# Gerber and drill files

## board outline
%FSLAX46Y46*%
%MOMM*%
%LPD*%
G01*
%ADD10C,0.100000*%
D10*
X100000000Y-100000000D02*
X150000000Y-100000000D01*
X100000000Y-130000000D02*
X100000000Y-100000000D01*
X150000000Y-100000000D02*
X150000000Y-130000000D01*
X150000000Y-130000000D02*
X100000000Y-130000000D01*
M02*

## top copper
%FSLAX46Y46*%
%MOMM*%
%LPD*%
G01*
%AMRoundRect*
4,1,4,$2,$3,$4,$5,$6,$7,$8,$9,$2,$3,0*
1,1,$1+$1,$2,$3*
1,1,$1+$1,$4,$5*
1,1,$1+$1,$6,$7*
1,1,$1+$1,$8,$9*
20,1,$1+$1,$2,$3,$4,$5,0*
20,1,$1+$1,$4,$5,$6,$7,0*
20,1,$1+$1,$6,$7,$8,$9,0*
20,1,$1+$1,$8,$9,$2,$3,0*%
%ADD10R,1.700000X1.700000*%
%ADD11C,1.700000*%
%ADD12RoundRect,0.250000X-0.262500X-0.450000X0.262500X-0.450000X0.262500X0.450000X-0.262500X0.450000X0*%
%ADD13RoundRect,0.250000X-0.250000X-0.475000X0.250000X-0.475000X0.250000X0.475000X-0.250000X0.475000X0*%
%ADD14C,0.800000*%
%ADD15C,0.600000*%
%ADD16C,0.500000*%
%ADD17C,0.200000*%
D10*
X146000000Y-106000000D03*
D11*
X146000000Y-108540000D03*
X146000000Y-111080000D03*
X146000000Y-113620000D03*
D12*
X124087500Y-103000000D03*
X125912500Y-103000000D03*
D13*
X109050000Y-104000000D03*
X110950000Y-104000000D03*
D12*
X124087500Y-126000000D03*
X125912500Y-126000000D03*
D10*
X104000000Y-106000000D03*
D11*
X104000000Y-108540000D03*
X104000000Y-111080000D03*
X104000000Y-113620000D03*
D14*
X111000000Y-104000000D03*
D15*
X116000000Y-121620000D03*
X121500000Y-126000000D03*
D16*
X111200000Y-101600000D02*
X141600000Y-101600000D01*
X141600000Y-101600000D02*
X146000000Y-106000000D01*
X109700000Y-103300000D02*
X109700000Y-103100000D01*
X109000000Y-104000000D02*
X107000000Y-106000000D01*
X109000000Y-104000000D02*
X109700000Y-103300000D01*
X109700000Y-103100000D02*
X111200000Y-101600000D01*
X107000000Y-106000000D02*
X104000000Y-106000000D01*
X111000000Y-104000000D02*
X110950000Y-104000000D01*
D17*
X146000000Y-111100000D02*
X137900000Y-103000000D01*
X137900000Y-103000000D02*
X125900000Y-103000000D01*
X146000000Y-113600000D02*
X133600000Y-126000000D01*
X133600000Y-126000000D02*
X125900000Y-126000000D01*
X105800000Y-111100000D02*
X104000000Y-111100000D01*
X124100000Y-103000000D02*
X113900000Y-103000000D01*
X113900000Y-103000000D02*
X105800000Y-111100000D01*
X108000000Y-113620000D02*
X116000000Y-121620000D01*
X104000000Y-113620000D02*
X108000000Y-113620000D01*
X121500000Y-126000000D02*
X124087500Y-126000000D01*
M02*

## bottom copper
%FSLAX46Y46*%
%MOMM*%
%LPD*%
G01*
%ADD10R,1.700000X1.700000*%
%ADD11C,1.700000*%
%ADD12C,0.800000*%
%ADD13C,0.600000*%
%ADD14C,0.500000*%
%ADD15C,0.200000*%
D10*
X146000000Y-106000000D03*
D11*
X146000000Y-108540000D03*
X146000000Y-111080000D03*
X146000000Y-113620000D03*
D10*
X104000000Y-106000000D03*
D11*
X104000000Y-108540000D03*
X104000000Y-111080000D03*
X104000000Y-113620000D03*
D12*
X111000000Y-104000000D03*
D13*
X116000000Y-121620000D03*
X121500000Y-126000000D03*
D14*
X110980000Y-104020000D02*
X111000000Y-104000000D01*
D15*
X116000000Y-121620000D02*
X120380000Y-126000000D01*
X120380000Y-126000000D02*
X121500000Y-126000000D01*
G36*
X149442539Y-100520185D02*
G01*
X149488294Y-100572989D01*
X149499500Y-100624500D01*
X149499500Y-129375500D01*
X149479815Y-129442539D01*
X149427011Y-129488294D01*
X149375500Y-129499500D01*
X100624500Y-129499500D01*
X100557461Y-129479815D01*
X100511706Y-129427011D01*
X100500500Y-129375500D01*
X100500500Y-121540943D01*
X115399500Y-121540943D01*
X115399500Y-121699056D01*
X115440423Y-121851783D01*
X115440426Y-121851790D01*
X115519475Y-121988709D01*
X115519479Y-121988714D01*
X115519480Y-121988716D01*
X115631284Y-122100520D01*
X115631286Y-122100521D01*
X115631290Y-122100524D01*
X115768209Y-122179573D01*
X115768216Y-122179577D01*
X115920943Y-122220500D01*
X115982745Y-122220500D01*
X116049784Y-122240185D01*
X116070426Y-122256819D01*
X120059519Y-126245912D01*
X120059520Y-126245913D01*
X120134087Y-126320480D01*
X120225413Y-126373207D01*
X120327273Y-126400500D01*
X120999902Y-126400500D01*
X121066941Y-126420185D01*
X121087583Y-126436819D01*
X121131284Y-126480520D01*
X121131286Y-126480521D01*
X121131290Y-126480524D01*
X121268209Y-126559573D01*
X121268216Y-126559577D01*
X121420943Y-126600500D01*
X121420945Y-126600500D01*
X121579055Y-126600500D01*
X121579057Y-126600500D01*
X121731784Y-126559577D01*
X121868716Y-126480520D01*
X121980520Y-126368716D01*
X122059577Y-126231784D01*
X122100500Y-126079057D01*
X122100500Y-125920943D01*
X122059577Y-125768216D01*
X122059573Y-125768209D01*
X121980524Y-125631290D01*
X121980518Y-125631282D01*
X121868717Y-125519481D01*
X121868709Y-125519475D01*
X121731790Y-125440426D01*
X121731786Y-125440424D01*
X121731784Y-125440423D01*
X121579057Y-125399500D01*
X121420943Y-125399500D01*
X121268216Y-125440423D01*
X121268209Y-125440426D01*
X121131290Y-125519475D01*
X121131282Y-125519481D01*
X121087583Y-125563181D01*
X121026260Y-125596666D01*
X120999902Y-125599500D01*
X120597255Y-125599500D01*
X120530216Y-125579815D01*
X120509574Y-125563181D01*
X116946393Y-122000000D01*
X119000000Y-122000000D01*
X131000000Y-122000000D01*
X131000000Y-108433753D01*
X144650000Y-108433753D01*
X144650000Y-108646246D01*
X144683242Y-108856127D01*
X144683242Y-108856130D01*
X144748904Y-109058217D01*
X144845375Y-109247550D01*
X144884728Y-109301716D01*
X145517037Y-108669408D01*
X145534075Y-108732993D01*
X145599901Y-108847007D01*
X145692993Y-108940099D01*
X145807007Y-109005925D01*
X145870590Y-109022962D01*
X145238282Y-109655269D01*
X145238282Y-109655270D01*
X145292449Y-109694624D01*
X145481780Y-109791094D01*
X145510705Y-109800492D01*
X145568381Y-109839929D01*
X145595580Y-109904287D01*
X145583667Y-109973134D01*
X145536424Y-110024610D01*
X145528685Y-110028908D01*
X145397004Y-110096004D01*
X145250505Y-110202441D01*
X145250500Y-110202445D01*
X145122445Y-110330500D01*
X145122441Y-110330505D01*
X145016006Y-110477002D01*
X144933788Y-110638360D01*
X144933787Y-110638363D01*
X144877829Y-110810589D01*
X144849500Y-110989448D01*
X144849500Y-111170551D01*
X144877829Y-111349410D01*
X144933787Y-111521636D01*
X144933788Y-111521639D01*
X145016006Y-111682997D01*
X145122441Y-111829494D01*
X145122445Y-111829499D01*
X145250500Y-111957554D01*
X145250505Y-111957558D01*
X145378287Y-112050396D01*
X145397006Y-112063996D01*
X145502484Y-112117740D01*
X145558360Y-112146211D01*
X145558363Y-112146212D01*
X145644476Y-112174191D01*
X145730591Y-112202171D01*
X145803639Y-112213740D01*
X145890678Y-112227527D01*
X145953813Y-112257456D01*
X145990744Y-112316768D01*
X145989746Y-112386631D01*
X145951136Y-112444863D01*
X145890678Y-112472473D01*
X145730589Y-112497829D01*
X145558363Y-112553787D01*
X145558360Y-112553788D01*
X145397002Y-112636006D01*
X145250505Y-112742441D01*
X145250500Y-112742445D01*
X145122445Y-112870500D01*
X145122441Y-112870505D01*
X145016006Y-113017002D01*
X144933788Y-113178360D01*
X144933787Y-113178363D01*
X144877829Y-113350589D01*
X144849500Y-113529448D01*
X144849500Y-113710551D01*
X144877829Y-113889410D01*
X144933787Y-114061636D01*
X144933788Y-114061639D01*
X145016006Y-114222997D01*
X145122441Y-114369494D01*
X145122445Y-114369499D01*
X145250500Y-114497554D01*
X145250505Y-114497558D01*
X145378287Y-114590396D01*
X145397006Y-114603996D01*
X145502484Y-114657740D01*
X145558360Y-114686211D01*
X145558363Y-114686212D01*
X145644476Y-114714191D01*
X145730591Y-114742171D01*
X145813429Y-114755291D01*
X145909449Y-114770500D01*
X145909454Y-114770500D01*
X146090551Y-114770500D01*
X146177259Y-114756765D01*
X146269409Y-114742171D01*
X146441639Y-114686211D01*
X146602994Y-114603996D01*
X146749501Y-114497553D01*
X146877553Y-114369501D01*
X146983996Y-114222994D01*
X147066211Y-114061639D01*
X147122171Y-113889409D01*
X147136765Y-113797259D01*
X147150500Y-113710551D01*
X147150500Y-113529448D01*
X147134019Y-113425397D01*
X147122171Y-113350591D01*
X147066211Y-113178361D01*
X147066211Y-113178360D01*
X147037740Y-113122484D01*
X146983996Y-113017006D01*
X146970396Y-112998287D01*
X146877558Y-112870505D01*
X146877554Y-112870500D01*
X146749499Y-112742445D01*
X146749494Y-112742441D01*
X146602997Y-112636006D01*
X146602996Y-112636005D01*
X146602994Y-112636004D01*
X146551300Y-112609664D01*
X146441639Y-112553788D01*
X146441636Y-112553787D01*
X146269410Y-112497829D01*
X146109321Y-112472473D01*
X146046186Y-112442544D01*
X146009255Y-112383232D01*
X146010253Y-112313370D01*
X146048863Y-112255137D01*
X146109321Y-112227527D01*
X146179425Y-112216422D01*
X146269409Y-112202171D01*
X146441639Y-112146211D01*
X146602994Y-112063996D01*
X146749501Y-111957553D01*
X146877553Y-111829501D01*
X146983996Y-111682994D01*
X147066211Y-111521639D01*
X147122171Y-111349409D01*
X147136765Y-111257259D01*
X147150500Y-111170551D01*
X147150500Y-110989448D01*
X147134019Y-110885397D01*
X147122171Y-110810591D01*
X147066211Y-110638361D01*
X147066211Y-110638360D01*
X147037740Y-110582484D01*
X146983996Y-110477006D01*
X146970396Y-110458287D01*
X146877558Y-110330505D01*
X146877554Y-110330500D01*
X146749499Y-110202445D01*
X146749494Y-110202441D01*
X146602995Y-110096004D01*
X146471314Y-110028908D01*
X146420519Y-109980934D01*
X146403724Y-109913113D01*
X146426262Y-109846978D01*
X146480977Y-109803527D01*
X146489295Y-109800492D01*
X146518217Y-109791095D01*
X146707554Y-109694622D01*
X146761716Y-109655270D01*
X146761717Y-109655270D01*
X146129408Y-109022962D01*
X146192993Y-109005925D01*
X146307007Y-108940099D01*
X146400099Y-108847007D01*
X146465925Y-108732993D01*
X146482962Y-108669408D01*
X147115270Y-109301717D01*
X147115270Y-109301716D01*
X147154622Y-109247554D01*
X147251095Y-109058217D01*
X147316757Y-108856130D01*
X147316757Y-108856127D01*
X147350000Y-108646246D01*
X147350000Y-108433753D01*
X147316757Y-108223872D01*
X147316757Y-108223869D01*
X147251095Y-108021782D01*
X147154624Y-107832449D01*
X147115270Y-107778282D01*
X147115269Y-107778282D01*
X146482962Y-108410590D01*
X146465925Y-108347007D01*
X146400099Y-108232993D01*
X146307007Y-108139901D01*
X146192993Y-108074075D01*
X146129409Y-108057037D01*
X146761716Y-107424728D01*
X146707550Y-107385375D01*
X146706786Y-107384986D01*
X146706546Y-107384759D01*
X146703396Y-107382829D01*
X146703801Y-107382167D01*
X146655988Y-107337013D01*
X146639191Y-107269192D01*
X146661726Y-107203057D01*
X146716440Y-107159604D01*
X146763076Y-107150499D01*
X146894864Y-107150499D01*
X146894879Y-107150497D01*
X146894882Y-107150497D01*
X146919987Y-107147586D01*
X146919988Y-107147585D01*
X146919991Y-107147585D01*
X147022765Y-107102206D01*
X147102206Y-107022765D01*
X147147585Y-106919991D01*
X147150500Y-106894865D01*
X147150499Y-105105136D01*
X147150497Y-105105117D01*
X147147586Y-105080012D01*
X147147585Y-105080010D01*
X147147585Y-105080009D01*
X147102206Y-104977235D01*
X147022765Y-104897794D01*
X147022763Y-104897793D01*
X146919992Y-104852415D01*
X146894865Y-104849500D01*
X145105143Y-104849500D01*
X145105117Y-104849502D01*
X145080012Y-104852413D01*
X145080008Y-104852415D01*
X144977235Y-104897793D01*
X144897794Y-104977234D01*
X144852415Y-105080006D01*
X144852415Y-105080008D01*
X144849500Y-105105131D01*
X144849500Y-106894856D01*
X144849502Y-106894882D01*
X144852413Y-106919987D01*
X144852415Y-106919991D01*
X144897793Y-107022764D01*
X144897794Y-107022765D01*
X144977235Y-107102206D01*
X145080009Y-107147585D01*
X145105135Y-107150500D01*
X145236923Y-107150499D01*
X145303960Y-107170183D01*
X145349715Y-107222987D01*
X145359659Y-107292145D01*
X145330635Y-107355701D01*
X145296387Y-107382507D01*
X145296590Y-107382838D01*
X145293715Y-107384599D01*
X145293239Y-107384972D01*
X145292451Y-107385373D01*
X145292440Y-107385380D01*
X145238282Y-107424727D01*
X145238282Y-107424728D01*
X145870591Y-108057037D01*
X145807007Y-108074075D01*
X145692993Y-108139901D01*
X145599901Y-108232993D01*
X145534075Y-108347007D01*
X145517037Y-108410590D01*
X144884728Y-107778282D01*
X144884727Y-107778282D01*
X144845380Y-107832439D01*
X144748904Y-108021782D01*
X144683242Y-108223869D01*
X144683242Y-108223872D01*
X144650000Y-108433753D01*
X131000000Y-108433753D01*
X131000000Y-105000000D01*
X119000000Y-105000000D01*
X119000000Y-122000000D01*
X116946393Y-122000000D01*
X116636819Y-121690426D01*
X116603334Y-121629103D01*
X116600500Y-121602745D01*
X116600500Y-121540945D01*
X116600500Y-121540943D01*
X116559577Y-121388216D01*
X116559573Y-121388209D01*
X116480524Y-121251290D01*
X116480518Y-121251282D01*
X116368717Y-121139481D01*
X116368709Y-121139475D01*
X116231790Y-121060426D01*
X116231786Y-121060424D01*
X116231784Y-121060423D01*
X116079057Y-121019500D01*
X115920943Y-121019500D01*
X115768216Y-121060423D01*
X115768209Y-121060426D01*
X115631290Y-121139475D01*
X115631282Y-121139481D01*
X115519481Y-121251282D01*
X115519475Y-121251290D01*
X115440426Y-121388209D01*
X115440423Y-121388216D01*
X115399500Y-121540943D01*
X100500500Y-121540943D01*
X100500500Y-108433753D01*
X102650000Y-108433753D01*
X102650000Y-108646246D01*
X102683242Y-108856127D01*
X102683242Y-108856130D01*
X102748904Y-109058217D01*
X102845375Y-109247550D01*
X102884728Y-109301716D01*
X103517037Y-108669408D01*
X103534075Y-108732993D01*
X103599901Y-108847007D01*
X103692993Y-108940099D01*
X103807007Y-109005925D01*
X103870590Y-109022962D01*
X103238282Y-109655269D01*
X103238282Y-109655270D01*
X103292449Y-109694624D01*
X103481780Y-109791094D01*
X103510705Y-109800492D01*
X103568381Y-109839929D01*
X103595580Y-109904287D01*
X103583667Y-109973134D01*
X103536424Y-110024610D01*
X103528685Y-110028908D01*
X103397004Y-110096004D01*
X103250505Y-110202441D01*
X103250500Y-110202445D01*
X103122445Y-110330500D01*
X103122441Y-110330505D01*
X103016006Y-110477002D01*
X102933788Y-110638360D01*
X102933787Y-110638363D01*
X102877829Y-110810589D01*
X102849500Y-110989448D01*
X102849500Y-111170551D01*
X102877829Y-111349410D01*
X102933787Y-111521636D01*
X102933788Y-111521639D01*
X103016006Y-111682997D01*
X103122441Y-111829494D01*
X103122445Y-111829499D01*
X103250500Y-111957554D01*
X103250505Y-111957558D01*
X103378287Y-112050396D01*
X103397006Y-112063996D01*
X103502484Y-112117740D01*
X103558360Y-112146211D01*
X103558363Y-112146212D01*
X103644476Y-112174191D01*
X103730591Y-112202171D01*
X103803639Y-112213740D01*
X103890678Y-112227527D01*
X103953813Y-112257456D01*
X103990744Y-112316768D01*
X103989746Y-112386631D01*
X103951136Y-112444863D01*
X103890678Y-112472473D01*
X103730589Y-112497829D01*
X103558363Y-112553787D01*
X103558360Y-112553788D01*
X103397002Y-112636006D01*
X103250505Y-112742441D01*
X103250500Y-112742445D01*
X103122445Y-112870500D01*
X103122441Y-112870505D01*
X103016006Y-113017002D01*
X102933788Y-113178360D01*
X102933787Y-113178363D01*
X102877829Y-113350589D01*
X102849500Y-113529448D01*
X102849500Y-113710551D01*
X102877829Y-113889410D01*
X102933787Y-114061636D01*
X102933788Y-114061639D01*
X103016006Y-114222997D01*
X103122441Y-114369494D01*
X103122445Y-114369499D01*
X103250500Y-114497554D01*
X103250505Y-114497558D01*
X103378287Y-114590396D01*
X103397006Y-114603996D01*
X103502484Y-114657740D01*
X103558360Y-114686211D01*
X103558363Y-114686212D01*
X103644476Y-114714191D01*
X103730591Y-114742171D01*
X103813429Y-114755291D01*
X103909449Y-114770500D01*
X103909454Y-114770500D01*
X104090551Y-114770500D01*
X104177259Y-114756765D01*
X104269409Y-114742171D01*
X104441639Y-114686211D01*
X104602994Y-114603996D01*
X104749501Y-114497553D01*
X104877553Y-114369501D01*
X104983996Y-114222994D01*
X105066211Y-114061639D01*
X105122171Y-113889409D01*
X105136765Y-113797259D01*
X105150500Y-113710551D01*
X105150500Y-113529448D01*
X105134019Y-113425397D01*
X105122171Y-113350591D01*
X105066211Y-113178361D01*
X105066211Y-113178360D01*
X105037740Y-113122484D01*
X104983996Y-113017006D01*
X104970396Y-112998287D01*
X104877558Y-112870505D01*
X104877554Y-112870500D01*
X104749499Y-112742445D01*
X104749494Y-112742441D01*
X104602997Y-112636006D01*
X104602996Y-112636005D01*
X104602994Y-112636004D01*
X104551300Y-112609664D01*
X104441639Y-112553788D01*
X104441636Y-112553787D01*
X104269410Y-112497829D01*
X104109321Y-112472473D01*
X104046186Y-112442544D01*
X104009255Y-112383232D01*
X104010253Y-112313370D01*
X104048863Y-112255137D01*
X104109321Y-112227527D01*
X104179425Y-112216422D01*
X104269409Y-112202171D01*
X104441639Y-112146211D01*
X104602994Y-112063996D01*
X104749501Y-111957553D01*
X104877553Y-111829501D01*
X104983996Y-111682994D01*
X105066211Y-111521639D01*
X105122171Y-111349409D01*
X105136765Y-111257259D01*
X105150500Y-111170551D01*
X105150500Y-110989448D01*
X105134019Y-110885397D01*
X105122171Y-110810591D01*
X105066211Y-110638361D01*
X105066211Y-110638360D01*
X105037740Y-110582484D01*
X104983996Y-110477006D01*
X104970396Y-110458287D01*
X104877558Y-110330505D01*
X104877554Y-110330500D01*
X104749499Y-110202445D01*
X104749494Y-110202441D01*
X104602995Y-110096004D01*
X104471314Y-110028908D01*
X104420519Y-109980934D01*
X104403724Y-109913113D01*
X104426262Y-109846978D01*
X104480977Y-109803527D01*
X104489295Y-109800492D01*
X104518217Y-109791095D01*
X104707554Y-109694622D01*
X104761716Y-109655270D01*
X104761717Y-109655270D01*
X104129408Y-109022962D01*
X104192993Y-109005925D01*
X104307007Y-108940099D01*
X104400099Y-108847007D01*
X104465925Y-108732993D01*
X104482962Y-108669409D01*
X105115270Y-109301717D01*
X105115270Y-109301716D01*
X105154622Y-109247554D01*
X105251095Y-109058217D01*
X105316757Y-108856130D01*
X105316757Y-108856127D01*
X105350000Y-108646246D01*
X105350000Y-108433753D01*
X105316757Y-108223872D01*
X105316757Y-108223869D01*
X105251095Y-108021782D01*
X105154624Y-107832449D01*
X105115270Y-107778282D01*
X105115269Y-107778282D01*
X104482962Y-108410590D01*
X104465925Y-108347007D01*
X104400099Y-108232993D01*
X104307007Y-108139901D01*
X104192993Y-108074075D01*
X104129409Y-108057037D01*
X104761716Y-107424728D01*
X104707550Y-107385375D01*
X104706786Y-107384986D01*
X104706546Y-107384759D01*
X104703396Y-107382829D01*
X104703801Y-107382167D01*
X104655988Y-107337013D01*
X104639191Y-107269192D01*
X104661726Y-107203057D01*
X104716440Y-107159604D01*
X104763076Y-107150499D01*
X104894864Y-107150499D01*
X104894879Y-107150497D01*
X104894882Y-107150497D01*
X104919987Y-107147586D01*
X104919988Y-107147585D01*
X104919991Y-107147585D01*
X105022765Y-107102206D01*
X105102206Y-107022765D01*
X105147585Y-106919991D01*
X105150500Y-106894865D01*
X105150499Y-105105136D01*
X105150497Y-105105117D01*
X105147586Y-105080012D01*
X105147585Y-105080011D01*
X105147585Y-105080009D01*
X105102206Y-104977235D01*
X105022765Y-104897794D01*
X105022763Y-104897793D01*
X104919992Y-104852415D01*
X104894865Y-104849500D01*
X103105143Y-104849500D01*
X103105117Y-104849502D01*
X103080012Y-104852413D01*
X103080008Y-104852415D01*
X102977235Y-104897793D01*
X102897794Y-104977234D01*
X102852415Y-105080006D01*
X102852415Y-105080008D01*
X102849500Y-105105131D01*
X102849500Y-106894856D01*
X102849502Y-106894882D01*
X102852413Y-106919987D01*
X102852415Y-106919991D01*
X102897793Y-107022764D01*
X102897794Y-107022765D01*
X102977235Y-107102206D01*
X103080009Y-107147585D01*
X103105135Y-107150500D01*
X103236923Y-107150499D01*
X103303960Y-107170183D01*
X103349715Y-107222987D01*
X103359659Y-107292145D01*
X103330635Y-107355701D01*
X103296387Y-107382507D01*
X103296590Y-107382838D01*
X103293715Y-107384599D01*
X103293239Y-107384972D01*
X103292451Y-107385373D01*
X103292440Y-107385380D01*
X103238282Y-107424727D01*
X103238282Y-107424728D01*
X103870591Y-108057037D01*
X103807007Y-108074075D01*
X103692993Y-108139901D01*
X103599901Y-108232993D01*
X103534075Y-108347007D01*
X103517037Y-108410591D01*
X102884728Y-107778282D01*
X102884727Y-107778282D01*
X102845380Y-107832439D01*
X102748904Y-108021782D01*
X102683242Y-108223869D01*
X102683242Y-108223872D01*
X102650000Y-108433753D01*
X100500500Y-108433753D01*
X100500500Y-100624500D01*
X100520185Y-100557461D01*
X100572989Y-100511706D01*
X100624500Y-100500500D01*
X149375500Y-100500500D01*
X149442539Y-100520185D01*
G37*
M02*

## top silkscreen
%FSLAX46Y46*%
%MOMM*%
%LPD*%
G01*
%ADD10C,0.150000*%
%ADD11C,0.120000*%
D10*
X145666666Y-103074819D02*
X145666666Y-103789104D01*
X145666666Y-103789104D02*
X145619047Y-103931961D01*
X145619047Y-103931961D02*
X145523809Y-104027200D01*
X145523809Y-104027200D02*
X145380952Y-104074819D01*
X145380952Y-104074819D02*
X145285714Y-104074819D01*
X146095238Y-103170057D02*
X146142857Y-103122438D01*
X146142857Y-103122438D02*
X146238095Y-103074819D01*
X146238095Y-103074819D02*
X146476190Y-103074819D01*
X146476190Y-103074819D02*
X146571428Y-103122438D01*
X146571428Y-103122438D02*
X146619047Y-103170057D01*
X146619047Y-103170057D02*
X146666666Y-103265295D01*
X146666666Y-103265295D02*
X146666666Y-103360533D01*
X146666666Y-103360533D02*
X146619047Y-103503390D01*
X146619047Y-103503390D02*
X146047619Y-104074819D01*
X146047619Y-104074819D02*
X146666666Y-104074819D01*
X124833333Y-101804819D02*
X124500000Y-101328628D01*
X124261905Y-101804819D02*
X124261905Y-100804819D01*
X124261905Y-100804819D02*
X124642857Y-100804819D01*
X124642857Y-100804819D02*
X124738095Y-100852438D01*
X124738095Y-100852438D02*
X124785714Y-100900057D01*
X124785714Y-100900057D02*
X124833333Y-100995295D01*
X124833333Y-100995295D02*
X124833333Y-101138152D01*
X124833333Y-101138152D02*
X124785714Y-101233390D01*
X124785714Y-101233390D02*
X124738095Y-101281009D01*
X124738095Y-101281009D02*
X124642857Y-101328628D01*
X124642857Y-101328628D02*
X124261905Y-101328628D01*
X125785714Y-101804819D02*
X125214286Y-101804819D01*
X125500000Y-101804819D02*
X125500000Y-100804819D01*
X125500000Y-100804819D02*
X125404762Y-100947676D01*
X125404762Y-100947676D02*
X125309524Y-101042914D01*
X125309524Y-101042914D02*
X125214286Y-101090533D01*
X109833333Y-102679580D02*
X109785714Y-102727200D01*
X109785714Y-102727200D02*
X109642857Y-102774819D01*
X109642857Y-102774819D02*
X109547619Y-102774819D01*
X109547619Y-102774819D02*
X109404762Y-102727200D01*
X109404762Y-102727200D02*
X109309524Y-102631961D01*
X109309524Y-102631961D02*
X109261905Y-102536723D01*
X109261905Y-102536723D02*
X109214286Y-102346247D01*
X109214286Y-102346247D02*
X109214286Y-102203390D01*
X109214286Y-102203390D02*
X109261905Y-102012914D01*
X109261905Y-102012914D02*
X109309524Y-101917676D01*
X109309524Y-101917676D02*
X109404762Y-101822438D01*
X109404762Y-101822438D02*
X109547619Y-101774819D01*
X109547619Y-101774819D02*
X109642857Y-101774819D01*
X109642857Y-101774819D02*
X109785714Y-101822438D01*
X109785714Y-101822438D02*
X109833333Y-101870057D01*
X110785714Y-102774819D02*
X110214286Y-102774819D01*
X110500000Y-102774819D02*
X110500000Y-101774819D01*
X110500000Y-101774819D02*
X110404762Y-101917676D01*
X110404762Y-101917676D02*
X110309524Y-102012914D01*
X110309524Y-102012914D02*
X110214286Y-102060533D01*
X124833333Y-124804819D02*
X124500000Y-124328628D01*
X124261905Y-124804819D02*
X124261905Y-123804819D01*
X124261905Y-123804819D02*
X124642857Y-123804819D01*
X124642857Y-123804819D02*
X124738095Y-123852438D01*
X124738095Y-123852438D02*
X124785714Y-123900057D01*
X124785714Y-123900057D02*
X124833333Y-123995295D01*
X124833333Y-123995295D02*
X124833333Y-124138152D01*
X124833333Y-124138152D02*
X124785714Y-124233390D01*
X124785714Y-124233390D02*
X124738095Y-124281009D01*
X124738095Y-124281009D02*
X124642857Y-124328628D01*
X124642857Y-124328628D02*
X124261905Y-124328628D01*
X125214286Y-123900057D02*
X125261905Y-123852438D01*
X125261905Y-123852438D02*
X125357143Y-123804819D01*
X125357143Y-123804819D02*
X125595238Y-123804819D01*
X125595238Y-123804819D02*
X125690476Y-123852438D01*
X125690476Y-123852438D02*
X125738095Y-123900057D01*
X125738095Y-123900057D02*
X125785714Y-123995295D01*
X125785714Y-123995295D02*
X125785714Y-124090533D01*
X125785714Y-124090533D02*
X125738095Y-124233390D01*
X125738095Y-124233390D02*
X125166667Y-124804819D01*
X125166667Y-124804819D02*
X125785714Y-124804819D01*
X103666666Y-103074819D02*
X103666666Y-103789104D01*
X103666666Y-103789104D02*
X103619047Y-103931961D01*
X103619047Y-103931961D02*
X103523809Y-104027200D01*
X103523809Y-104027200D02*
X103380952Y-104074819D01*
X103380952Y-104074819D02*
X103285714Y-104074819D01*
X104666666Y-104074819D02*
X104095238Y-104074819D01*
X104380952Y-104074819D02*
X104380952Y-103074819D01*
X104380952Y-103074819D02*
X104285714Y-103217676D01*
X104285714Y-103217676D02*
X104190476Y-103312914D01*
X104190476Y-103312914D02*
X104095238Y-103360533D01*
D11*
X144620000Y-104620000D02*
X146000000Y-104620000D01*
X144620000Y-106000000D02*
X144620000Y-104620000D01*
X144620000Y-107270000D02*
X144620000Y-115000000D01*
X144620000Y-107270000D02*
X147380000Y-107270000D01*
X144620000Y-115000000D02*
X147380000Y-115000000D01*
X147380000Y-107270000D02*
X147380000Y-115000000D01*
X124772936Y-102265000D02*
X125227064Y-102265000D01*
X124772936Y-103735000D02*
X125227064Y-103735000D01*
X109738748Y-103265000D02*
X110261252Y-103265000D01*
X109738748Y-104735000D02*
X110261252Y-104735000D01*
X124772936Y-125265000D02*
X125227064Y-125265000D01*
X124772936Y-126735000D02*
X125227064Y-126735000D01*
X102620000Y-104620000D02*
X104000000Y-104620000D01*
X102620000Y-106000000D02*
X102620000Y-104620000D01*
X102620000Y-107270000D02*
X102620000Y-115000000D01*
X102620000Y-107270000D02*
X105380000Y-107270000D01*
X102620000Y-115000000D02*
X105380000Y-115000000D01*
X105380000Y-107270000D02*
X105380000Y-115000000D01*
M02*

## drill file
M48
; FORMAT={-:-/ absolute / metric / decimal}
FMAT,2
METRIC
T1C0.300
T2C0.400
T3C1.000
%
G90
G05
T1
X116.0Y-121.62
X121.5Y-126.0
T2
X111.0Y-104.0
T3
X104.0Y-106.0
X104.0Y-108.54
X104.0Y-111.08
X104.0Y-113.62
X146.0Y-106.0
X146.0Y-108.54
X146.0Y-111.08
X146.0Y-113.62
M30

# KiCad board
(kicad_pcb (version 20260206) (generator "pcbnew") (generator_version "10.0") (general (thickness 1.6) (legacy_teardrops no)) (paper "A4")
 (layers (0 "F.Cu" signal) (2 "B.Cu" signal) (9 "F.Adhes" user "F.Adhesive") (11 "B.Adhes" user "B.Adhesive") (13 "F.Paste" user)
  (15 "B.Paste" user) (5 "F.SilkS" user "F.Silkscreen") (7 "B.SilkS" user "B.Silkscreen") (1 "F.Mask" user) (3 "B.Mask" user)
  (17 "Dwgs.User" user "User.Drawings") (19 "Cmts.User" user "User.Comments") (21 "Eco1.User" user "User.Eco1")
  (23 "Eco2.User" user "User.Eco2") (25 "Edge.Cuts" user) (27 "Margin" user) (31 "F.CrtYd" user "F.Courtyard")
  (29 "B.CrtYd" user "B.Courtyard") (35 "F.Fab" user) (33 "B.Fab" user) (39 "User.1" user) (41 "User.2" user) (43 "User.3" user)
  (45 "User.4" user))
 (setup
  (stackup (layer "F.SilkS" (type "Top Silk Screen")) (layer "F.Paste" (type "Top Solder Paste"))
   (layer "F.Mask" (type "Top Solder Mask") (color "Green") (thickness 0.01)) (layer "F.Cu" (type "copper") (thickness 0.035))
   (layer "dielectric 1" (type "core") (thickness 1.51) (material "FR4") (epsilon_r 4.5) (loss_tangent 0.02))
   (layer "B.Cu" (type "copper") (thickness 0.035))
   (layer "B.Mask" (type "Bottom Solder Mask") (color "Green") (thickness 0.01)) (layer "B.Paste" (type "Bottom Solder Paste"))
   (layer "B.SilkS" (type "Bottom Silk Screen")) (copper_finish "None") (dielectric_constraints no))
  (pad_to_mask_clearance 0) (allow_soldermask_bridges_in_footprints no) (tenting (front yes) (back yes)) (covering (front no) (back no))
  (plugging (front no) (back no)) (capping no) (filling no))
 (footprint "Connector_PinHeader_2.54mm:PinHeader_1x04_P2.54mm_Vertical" (layer "F.Cu") (at 146 106)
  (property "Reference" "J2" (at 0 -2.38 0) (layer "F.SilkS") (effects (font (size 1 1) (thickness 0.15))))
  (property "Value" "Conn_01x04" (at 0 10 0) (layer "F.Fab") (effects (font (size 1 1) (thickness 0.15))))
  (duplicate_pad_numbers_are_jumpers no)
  (fp_line (start -1.38 -1.38) (end 0 -1.38) (stroke (width 0.12) (type solid)) (layer "F.SilkS"))
  (fp_line (start -1.38 0) (end -1.38 -1.38) (stroke (width 0.12) (type solid)) (layer "F.SilkS"))
  (fp_line (start -1.38 1.27) (end -1.38 9) (stroke (width 0.12) (type solid)) (layer "F.SilkS"))
  (fp_line (start -1.38 1.27) (end 1.38 1.27) (stroke (width 0.12) (type solid)) (layer "F.SilkS"))
  (fp_line (start -1.38 9) (end 1.38 9) (stroke (width 0.12) (type solid)) (layer "F.SilkS"))
  (fp_line (start 1.38 1.27) (end 1.38 9) (stroke (width 0.12) (type solid)) (layer "F.SilkS"))
  (pad "1" thru_hole rect (at 0 0) (size 1.7 1.7) (drill 1) (layers "*.Cu" "*.Mask") (remove_unused_layers no) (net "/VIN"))
  (pad "2" thru_hole circle (at 0 2.54) (size 1.7 1.7) (drill 1) (layers "*.Cu" "*.Mask") (remove_unused_layers no) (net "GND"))
  (pad "3" thru_hole circle (at 0 5.08) (size 1.7 1.7) (drill 1) (layers "*.Cu" "*.Mask") (remove_unused_layers no) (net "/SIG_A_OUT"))
  (pad "4" thru_hole circle (at 0 7.62) (size 1.7 1.7) (drill 1) (layers "*.Cu" "*.Mask") (remove_unused_layers no) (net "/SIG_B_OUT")))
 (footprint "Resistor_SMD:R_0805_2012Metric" (layer "F.Cu") (at 125 103)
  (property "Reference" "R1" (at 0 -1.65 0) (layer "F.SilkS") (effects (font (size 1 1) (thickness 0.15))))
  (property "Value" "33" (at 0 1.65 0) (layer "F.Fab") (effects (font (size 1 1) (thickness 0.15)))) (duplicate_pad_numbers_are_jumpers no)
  (fp_line (start -0.227064 -0.735) (end 0.227064 -0.735) (stroke (width 0.12) (type solid)) (layer "F.SilkS"))
  (fp_line (start -0.227064 0.735) (end 0.227064 0.735) (stroke (width 0.12) (type solid)) (layer "F.SilkS"))
  (pad "1" smd roundrect (at -0.9125 0) (size 1.025 1.4) (layers "F.Cu" "F.Mask" "F.Paste") (roundrect_rratio 0.243902) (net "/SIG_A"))
  (pad "2" smd roundrect (at 0.9125 0) (size 1.025 1.4) (layers "F.Cu" "F.Mask" "F.Paste") (roundrect_rratio 0.243902) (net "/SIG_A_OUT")))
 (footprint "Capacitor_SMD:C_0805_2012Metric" (layer "F.Cu") (at 110 104)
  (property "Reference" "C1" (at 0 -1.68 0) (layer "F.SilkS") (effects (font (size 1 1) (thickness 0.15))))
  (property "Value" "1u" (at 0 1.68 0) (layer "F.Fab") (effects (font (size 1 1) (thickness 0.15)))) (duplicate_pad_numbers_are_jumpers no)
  (fp_line (start -0.261252 -0.735) (end 0.261252 -0.735) (stroke (width 0.12) (type solid)) (layer "F.SilkS"))
  (fp_line (start -0.261252 0.735) (end 0.261252 0.735) (stroke (width 0.12) (type solid)) (layer "F.SilkS"))
  (pad "1" smd roundrect (at -0.95 0) (size 1 1.45) (layers "F.Cu" "F.Mask" "F.Paste") (roundrect_rratio 0.25) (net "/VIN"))
  (pad "2" smd roundrect (at 0.95 0) (size 1 1.45) (layers "F.Cu" "F.Mask" "F.Paste") (roundrect_rratio 0.25) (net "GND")))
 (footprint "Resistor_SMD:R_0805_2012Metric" (layer "F.Cu") (at 125 126)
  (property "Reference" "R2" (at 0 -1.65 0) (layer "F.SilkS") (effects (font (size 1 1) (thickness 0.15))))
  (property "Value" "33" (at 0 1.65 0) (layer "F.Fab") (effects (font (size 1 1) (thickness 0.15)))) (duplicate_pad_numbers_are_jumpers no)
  (fp_line (start -0.227064 -0.735) (end 0.227064 -0.735) (stroke (width 0.12) (type solid)) (layer "F.SilkS"))
  (fp_line (start -0.227064 0.735) (end 0.227064 0.735) (stroke (width 0.12) (type solid)) (layer "F.SilkS"))
  (pad "1" smd roundrect (at -0.9125 0) (size 1.025 1.4) (layers "F.Cu" "F.Mask" "F.Paste") (roundrect_rratio 0.243902) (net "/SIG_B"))
  (pad "2" smd roundrect (at 0.9125 0) (size 1.025 1.4) (layers "F.Cu" "F.Mask" "F.Paste") (roundrect_rratio 0.243902) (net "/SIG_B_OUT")))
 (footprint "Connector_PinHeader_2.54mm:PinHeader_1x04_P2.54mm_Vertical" (layer "F.Cu") (at 104 106)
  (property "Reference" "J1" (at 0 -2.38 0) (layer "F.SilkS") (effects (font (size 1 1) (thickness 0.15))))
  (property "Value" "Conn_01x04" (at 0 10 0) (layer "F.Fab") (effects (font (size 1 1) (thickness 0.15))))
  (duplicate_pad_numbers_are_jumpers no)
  (fp_line (start -1.38 -1.38) (end 0 -1.38) (stroke (width 0.12) (type solid)) (layer "F.SilkS"))
  (fp_line (start -1.38 0) (end -1.38 -1.38) (stroke (width 0.12) (type solid)) (layer "F.SilkS"))
  (fp_line (start -1.38 1.27) (end -1.38 9) (stroke (width 0.12) (type solid)) (layer "F.SilkS"))
  (fp_line (start -1.38 1.27) (end 1.38 1.27) (stroke (width 0.12) (type solid)) (layer "F.SilkS"))
  (fp_line (start -1.38 9) (end 1.38 9) (stroke (width 0.12) (type solid)) (layer "F.SilkS"))
  (fp_line (start 1.38 1.27) (end 1.38 9) (stroke (width 0.12) (type solid)) (layer "F.SilkS"))
  (pad "1" thru_hole rect (at 0 0) (size 1.7 1.7) (drill 1) (layers "*.Cu" "*.Mask") (remove_unused_layers no) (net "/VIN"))
  (pad "2" thru_hole circle (at 0 2.54) (size 1.7 1.7) (drill 1) (layers "*.Cu" "*.Mask") (remove_unused_layers no) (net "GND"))
  (pad "3" thru_hole circle (at 0 5.08) (size 1.7 1.7) (drill 1) (layers "*.Cu" "*.Mask") (remove_unused_layers no) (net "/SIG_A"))
  (pad "4" thru_hole circle (at 0 7.62) (size 1.7 1.7) (drill 1) (layers "*.Cu" "*.Mask") (remove_unused_layers no) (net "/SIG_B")))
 (gr_line (start 100 100) (end 150 100) (stroke (width 0.1) (type default)) (layer "Edge.Cuts"))
 (gr_line (start 100 130) (end 100 100) (stroke (width 0.1) (type default)) (layer "Edge.Cuts"))
 (gr_line (start 150 100) (end 150 130) (stroke (width 0.1) (type default)) (layer "Edge.Cuts"))
 (gr_line (start 150 130) (end 100 130) (stroke (width 0.1) (type default)) (layer "Edge.Cuts"))
 (segment (start 111.2 101.6) (end 141.6 101.6) (width 0.5) (layer "F.Cu") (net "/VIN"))
 (segment (start 141.6 101.6) (end 146 106) (width 0.5) (layer "F.Cu") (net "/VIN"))
 (segment (start 109.7 103.3) (end 109.7 103.1) (width 0.5) (layer "F.Cu") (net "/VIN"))
 (segment (start 109 104) (end 107 106) (width 0.5) (layer "F.Cu") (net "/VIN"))
 (segment (start 109 104) (end 109.7 103.3) (width 0.5) (layer "F.Cu") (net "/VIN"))
 (segment (start 109.7 103.1) (end 111.2 101.6) (width 0.5) (layer "F.Cu") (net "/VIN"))
 (segment (start 107 106) (end 104 106) (width 0.5) (layer "F.Cu") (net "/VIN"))
 (segment (start 111 104) (end 110.95 104) (width 0.5) (layer "F.Cu") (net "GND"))
 (via (at 111 104) (size 0.8) (drill 0.4) (layers "F.Cu" "B.Cu") (capping yes) (filling yes) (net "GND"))
 (segment (start 110.98 104.02) (end 111 104) (width 0.5) (layer "B.Cu") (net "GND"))
 (segment (start 146 111.1) (end 137.9 103) (width 0.2) (layer "F.Cu") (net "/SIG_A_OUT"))
 (segment (start 137.9 103) (end 125.9 103) (width 0.2) (layer "F.Cu") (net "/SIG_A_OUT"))
 (segment (start 146 113.6) (end 133.6 126) (width 0.2) (layer "F.Cu") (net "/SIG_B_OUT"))
 (segment (start 133.6 126) (end 125.9 126) (width 0.2) (layer "F.Cu") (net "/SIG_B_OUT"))
 (segment (start 105.8 111.1) (end 104 111.1) (width 0.2) (layer "F.Cu") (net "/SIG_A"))
 (segment (start 124.1 103) (end 113.9 103) (width 0.2) (layer "F.Cu") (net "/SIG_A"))
 (segment (start 113.9 103) (end 105.8 111.1) (width 0.2) (layer "F.Cu") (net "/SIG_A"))
 (segment (start 108 113.62) (end 116 121.62) (width 0.2) (locked yes) (layer "F.Cu") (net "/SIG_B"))
 (segment (start 104 113.62) (end 108 113.62) (width 0.2) (locked yes) (layer "F.Cu") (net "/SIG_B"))
 (segment (start 121.5 126) (end 124.0875 126) (width 0.2) (locked yes) (layer "F.Cu") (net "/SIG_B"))
 (via (at 116 121.62) (size 0.6) (drill 0.3) (layers "F.Cu" "B.Cu") (locked yes) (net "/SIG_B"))
 (via (at 121.5 126) (size 0.6) (drill 0.3) (layers "F.Cu" "B.Cu") (locked yes) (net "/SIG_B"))
 (segment (start 116 121.62) (end 120.38 126) (width 0.2) (locked yes) (layer "B.Cu") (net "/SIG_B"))
 (segment (start 120.38 126) (end 121.5 126) (width 0.2) (locked yes) (layer "B.Cu") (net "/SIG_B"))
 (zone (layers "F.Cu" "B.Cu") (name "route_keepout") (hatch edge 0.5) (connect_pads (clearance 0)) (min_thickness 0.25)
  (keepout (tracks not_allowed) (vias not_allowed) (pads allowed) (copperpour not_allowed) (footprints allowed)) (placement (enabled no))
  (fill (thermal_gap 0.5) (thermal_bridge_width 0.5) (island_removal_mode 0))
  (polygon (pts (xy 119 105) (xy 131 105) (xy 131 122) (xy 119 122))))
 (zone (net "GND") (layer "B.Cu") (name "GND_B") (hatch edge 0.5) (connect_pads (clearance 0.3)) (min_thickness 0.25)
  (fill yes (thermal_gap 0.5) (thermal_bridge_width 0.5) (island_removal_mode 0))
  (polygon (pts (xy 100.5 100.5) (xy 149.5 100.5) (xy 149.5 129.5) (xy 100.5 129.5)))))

